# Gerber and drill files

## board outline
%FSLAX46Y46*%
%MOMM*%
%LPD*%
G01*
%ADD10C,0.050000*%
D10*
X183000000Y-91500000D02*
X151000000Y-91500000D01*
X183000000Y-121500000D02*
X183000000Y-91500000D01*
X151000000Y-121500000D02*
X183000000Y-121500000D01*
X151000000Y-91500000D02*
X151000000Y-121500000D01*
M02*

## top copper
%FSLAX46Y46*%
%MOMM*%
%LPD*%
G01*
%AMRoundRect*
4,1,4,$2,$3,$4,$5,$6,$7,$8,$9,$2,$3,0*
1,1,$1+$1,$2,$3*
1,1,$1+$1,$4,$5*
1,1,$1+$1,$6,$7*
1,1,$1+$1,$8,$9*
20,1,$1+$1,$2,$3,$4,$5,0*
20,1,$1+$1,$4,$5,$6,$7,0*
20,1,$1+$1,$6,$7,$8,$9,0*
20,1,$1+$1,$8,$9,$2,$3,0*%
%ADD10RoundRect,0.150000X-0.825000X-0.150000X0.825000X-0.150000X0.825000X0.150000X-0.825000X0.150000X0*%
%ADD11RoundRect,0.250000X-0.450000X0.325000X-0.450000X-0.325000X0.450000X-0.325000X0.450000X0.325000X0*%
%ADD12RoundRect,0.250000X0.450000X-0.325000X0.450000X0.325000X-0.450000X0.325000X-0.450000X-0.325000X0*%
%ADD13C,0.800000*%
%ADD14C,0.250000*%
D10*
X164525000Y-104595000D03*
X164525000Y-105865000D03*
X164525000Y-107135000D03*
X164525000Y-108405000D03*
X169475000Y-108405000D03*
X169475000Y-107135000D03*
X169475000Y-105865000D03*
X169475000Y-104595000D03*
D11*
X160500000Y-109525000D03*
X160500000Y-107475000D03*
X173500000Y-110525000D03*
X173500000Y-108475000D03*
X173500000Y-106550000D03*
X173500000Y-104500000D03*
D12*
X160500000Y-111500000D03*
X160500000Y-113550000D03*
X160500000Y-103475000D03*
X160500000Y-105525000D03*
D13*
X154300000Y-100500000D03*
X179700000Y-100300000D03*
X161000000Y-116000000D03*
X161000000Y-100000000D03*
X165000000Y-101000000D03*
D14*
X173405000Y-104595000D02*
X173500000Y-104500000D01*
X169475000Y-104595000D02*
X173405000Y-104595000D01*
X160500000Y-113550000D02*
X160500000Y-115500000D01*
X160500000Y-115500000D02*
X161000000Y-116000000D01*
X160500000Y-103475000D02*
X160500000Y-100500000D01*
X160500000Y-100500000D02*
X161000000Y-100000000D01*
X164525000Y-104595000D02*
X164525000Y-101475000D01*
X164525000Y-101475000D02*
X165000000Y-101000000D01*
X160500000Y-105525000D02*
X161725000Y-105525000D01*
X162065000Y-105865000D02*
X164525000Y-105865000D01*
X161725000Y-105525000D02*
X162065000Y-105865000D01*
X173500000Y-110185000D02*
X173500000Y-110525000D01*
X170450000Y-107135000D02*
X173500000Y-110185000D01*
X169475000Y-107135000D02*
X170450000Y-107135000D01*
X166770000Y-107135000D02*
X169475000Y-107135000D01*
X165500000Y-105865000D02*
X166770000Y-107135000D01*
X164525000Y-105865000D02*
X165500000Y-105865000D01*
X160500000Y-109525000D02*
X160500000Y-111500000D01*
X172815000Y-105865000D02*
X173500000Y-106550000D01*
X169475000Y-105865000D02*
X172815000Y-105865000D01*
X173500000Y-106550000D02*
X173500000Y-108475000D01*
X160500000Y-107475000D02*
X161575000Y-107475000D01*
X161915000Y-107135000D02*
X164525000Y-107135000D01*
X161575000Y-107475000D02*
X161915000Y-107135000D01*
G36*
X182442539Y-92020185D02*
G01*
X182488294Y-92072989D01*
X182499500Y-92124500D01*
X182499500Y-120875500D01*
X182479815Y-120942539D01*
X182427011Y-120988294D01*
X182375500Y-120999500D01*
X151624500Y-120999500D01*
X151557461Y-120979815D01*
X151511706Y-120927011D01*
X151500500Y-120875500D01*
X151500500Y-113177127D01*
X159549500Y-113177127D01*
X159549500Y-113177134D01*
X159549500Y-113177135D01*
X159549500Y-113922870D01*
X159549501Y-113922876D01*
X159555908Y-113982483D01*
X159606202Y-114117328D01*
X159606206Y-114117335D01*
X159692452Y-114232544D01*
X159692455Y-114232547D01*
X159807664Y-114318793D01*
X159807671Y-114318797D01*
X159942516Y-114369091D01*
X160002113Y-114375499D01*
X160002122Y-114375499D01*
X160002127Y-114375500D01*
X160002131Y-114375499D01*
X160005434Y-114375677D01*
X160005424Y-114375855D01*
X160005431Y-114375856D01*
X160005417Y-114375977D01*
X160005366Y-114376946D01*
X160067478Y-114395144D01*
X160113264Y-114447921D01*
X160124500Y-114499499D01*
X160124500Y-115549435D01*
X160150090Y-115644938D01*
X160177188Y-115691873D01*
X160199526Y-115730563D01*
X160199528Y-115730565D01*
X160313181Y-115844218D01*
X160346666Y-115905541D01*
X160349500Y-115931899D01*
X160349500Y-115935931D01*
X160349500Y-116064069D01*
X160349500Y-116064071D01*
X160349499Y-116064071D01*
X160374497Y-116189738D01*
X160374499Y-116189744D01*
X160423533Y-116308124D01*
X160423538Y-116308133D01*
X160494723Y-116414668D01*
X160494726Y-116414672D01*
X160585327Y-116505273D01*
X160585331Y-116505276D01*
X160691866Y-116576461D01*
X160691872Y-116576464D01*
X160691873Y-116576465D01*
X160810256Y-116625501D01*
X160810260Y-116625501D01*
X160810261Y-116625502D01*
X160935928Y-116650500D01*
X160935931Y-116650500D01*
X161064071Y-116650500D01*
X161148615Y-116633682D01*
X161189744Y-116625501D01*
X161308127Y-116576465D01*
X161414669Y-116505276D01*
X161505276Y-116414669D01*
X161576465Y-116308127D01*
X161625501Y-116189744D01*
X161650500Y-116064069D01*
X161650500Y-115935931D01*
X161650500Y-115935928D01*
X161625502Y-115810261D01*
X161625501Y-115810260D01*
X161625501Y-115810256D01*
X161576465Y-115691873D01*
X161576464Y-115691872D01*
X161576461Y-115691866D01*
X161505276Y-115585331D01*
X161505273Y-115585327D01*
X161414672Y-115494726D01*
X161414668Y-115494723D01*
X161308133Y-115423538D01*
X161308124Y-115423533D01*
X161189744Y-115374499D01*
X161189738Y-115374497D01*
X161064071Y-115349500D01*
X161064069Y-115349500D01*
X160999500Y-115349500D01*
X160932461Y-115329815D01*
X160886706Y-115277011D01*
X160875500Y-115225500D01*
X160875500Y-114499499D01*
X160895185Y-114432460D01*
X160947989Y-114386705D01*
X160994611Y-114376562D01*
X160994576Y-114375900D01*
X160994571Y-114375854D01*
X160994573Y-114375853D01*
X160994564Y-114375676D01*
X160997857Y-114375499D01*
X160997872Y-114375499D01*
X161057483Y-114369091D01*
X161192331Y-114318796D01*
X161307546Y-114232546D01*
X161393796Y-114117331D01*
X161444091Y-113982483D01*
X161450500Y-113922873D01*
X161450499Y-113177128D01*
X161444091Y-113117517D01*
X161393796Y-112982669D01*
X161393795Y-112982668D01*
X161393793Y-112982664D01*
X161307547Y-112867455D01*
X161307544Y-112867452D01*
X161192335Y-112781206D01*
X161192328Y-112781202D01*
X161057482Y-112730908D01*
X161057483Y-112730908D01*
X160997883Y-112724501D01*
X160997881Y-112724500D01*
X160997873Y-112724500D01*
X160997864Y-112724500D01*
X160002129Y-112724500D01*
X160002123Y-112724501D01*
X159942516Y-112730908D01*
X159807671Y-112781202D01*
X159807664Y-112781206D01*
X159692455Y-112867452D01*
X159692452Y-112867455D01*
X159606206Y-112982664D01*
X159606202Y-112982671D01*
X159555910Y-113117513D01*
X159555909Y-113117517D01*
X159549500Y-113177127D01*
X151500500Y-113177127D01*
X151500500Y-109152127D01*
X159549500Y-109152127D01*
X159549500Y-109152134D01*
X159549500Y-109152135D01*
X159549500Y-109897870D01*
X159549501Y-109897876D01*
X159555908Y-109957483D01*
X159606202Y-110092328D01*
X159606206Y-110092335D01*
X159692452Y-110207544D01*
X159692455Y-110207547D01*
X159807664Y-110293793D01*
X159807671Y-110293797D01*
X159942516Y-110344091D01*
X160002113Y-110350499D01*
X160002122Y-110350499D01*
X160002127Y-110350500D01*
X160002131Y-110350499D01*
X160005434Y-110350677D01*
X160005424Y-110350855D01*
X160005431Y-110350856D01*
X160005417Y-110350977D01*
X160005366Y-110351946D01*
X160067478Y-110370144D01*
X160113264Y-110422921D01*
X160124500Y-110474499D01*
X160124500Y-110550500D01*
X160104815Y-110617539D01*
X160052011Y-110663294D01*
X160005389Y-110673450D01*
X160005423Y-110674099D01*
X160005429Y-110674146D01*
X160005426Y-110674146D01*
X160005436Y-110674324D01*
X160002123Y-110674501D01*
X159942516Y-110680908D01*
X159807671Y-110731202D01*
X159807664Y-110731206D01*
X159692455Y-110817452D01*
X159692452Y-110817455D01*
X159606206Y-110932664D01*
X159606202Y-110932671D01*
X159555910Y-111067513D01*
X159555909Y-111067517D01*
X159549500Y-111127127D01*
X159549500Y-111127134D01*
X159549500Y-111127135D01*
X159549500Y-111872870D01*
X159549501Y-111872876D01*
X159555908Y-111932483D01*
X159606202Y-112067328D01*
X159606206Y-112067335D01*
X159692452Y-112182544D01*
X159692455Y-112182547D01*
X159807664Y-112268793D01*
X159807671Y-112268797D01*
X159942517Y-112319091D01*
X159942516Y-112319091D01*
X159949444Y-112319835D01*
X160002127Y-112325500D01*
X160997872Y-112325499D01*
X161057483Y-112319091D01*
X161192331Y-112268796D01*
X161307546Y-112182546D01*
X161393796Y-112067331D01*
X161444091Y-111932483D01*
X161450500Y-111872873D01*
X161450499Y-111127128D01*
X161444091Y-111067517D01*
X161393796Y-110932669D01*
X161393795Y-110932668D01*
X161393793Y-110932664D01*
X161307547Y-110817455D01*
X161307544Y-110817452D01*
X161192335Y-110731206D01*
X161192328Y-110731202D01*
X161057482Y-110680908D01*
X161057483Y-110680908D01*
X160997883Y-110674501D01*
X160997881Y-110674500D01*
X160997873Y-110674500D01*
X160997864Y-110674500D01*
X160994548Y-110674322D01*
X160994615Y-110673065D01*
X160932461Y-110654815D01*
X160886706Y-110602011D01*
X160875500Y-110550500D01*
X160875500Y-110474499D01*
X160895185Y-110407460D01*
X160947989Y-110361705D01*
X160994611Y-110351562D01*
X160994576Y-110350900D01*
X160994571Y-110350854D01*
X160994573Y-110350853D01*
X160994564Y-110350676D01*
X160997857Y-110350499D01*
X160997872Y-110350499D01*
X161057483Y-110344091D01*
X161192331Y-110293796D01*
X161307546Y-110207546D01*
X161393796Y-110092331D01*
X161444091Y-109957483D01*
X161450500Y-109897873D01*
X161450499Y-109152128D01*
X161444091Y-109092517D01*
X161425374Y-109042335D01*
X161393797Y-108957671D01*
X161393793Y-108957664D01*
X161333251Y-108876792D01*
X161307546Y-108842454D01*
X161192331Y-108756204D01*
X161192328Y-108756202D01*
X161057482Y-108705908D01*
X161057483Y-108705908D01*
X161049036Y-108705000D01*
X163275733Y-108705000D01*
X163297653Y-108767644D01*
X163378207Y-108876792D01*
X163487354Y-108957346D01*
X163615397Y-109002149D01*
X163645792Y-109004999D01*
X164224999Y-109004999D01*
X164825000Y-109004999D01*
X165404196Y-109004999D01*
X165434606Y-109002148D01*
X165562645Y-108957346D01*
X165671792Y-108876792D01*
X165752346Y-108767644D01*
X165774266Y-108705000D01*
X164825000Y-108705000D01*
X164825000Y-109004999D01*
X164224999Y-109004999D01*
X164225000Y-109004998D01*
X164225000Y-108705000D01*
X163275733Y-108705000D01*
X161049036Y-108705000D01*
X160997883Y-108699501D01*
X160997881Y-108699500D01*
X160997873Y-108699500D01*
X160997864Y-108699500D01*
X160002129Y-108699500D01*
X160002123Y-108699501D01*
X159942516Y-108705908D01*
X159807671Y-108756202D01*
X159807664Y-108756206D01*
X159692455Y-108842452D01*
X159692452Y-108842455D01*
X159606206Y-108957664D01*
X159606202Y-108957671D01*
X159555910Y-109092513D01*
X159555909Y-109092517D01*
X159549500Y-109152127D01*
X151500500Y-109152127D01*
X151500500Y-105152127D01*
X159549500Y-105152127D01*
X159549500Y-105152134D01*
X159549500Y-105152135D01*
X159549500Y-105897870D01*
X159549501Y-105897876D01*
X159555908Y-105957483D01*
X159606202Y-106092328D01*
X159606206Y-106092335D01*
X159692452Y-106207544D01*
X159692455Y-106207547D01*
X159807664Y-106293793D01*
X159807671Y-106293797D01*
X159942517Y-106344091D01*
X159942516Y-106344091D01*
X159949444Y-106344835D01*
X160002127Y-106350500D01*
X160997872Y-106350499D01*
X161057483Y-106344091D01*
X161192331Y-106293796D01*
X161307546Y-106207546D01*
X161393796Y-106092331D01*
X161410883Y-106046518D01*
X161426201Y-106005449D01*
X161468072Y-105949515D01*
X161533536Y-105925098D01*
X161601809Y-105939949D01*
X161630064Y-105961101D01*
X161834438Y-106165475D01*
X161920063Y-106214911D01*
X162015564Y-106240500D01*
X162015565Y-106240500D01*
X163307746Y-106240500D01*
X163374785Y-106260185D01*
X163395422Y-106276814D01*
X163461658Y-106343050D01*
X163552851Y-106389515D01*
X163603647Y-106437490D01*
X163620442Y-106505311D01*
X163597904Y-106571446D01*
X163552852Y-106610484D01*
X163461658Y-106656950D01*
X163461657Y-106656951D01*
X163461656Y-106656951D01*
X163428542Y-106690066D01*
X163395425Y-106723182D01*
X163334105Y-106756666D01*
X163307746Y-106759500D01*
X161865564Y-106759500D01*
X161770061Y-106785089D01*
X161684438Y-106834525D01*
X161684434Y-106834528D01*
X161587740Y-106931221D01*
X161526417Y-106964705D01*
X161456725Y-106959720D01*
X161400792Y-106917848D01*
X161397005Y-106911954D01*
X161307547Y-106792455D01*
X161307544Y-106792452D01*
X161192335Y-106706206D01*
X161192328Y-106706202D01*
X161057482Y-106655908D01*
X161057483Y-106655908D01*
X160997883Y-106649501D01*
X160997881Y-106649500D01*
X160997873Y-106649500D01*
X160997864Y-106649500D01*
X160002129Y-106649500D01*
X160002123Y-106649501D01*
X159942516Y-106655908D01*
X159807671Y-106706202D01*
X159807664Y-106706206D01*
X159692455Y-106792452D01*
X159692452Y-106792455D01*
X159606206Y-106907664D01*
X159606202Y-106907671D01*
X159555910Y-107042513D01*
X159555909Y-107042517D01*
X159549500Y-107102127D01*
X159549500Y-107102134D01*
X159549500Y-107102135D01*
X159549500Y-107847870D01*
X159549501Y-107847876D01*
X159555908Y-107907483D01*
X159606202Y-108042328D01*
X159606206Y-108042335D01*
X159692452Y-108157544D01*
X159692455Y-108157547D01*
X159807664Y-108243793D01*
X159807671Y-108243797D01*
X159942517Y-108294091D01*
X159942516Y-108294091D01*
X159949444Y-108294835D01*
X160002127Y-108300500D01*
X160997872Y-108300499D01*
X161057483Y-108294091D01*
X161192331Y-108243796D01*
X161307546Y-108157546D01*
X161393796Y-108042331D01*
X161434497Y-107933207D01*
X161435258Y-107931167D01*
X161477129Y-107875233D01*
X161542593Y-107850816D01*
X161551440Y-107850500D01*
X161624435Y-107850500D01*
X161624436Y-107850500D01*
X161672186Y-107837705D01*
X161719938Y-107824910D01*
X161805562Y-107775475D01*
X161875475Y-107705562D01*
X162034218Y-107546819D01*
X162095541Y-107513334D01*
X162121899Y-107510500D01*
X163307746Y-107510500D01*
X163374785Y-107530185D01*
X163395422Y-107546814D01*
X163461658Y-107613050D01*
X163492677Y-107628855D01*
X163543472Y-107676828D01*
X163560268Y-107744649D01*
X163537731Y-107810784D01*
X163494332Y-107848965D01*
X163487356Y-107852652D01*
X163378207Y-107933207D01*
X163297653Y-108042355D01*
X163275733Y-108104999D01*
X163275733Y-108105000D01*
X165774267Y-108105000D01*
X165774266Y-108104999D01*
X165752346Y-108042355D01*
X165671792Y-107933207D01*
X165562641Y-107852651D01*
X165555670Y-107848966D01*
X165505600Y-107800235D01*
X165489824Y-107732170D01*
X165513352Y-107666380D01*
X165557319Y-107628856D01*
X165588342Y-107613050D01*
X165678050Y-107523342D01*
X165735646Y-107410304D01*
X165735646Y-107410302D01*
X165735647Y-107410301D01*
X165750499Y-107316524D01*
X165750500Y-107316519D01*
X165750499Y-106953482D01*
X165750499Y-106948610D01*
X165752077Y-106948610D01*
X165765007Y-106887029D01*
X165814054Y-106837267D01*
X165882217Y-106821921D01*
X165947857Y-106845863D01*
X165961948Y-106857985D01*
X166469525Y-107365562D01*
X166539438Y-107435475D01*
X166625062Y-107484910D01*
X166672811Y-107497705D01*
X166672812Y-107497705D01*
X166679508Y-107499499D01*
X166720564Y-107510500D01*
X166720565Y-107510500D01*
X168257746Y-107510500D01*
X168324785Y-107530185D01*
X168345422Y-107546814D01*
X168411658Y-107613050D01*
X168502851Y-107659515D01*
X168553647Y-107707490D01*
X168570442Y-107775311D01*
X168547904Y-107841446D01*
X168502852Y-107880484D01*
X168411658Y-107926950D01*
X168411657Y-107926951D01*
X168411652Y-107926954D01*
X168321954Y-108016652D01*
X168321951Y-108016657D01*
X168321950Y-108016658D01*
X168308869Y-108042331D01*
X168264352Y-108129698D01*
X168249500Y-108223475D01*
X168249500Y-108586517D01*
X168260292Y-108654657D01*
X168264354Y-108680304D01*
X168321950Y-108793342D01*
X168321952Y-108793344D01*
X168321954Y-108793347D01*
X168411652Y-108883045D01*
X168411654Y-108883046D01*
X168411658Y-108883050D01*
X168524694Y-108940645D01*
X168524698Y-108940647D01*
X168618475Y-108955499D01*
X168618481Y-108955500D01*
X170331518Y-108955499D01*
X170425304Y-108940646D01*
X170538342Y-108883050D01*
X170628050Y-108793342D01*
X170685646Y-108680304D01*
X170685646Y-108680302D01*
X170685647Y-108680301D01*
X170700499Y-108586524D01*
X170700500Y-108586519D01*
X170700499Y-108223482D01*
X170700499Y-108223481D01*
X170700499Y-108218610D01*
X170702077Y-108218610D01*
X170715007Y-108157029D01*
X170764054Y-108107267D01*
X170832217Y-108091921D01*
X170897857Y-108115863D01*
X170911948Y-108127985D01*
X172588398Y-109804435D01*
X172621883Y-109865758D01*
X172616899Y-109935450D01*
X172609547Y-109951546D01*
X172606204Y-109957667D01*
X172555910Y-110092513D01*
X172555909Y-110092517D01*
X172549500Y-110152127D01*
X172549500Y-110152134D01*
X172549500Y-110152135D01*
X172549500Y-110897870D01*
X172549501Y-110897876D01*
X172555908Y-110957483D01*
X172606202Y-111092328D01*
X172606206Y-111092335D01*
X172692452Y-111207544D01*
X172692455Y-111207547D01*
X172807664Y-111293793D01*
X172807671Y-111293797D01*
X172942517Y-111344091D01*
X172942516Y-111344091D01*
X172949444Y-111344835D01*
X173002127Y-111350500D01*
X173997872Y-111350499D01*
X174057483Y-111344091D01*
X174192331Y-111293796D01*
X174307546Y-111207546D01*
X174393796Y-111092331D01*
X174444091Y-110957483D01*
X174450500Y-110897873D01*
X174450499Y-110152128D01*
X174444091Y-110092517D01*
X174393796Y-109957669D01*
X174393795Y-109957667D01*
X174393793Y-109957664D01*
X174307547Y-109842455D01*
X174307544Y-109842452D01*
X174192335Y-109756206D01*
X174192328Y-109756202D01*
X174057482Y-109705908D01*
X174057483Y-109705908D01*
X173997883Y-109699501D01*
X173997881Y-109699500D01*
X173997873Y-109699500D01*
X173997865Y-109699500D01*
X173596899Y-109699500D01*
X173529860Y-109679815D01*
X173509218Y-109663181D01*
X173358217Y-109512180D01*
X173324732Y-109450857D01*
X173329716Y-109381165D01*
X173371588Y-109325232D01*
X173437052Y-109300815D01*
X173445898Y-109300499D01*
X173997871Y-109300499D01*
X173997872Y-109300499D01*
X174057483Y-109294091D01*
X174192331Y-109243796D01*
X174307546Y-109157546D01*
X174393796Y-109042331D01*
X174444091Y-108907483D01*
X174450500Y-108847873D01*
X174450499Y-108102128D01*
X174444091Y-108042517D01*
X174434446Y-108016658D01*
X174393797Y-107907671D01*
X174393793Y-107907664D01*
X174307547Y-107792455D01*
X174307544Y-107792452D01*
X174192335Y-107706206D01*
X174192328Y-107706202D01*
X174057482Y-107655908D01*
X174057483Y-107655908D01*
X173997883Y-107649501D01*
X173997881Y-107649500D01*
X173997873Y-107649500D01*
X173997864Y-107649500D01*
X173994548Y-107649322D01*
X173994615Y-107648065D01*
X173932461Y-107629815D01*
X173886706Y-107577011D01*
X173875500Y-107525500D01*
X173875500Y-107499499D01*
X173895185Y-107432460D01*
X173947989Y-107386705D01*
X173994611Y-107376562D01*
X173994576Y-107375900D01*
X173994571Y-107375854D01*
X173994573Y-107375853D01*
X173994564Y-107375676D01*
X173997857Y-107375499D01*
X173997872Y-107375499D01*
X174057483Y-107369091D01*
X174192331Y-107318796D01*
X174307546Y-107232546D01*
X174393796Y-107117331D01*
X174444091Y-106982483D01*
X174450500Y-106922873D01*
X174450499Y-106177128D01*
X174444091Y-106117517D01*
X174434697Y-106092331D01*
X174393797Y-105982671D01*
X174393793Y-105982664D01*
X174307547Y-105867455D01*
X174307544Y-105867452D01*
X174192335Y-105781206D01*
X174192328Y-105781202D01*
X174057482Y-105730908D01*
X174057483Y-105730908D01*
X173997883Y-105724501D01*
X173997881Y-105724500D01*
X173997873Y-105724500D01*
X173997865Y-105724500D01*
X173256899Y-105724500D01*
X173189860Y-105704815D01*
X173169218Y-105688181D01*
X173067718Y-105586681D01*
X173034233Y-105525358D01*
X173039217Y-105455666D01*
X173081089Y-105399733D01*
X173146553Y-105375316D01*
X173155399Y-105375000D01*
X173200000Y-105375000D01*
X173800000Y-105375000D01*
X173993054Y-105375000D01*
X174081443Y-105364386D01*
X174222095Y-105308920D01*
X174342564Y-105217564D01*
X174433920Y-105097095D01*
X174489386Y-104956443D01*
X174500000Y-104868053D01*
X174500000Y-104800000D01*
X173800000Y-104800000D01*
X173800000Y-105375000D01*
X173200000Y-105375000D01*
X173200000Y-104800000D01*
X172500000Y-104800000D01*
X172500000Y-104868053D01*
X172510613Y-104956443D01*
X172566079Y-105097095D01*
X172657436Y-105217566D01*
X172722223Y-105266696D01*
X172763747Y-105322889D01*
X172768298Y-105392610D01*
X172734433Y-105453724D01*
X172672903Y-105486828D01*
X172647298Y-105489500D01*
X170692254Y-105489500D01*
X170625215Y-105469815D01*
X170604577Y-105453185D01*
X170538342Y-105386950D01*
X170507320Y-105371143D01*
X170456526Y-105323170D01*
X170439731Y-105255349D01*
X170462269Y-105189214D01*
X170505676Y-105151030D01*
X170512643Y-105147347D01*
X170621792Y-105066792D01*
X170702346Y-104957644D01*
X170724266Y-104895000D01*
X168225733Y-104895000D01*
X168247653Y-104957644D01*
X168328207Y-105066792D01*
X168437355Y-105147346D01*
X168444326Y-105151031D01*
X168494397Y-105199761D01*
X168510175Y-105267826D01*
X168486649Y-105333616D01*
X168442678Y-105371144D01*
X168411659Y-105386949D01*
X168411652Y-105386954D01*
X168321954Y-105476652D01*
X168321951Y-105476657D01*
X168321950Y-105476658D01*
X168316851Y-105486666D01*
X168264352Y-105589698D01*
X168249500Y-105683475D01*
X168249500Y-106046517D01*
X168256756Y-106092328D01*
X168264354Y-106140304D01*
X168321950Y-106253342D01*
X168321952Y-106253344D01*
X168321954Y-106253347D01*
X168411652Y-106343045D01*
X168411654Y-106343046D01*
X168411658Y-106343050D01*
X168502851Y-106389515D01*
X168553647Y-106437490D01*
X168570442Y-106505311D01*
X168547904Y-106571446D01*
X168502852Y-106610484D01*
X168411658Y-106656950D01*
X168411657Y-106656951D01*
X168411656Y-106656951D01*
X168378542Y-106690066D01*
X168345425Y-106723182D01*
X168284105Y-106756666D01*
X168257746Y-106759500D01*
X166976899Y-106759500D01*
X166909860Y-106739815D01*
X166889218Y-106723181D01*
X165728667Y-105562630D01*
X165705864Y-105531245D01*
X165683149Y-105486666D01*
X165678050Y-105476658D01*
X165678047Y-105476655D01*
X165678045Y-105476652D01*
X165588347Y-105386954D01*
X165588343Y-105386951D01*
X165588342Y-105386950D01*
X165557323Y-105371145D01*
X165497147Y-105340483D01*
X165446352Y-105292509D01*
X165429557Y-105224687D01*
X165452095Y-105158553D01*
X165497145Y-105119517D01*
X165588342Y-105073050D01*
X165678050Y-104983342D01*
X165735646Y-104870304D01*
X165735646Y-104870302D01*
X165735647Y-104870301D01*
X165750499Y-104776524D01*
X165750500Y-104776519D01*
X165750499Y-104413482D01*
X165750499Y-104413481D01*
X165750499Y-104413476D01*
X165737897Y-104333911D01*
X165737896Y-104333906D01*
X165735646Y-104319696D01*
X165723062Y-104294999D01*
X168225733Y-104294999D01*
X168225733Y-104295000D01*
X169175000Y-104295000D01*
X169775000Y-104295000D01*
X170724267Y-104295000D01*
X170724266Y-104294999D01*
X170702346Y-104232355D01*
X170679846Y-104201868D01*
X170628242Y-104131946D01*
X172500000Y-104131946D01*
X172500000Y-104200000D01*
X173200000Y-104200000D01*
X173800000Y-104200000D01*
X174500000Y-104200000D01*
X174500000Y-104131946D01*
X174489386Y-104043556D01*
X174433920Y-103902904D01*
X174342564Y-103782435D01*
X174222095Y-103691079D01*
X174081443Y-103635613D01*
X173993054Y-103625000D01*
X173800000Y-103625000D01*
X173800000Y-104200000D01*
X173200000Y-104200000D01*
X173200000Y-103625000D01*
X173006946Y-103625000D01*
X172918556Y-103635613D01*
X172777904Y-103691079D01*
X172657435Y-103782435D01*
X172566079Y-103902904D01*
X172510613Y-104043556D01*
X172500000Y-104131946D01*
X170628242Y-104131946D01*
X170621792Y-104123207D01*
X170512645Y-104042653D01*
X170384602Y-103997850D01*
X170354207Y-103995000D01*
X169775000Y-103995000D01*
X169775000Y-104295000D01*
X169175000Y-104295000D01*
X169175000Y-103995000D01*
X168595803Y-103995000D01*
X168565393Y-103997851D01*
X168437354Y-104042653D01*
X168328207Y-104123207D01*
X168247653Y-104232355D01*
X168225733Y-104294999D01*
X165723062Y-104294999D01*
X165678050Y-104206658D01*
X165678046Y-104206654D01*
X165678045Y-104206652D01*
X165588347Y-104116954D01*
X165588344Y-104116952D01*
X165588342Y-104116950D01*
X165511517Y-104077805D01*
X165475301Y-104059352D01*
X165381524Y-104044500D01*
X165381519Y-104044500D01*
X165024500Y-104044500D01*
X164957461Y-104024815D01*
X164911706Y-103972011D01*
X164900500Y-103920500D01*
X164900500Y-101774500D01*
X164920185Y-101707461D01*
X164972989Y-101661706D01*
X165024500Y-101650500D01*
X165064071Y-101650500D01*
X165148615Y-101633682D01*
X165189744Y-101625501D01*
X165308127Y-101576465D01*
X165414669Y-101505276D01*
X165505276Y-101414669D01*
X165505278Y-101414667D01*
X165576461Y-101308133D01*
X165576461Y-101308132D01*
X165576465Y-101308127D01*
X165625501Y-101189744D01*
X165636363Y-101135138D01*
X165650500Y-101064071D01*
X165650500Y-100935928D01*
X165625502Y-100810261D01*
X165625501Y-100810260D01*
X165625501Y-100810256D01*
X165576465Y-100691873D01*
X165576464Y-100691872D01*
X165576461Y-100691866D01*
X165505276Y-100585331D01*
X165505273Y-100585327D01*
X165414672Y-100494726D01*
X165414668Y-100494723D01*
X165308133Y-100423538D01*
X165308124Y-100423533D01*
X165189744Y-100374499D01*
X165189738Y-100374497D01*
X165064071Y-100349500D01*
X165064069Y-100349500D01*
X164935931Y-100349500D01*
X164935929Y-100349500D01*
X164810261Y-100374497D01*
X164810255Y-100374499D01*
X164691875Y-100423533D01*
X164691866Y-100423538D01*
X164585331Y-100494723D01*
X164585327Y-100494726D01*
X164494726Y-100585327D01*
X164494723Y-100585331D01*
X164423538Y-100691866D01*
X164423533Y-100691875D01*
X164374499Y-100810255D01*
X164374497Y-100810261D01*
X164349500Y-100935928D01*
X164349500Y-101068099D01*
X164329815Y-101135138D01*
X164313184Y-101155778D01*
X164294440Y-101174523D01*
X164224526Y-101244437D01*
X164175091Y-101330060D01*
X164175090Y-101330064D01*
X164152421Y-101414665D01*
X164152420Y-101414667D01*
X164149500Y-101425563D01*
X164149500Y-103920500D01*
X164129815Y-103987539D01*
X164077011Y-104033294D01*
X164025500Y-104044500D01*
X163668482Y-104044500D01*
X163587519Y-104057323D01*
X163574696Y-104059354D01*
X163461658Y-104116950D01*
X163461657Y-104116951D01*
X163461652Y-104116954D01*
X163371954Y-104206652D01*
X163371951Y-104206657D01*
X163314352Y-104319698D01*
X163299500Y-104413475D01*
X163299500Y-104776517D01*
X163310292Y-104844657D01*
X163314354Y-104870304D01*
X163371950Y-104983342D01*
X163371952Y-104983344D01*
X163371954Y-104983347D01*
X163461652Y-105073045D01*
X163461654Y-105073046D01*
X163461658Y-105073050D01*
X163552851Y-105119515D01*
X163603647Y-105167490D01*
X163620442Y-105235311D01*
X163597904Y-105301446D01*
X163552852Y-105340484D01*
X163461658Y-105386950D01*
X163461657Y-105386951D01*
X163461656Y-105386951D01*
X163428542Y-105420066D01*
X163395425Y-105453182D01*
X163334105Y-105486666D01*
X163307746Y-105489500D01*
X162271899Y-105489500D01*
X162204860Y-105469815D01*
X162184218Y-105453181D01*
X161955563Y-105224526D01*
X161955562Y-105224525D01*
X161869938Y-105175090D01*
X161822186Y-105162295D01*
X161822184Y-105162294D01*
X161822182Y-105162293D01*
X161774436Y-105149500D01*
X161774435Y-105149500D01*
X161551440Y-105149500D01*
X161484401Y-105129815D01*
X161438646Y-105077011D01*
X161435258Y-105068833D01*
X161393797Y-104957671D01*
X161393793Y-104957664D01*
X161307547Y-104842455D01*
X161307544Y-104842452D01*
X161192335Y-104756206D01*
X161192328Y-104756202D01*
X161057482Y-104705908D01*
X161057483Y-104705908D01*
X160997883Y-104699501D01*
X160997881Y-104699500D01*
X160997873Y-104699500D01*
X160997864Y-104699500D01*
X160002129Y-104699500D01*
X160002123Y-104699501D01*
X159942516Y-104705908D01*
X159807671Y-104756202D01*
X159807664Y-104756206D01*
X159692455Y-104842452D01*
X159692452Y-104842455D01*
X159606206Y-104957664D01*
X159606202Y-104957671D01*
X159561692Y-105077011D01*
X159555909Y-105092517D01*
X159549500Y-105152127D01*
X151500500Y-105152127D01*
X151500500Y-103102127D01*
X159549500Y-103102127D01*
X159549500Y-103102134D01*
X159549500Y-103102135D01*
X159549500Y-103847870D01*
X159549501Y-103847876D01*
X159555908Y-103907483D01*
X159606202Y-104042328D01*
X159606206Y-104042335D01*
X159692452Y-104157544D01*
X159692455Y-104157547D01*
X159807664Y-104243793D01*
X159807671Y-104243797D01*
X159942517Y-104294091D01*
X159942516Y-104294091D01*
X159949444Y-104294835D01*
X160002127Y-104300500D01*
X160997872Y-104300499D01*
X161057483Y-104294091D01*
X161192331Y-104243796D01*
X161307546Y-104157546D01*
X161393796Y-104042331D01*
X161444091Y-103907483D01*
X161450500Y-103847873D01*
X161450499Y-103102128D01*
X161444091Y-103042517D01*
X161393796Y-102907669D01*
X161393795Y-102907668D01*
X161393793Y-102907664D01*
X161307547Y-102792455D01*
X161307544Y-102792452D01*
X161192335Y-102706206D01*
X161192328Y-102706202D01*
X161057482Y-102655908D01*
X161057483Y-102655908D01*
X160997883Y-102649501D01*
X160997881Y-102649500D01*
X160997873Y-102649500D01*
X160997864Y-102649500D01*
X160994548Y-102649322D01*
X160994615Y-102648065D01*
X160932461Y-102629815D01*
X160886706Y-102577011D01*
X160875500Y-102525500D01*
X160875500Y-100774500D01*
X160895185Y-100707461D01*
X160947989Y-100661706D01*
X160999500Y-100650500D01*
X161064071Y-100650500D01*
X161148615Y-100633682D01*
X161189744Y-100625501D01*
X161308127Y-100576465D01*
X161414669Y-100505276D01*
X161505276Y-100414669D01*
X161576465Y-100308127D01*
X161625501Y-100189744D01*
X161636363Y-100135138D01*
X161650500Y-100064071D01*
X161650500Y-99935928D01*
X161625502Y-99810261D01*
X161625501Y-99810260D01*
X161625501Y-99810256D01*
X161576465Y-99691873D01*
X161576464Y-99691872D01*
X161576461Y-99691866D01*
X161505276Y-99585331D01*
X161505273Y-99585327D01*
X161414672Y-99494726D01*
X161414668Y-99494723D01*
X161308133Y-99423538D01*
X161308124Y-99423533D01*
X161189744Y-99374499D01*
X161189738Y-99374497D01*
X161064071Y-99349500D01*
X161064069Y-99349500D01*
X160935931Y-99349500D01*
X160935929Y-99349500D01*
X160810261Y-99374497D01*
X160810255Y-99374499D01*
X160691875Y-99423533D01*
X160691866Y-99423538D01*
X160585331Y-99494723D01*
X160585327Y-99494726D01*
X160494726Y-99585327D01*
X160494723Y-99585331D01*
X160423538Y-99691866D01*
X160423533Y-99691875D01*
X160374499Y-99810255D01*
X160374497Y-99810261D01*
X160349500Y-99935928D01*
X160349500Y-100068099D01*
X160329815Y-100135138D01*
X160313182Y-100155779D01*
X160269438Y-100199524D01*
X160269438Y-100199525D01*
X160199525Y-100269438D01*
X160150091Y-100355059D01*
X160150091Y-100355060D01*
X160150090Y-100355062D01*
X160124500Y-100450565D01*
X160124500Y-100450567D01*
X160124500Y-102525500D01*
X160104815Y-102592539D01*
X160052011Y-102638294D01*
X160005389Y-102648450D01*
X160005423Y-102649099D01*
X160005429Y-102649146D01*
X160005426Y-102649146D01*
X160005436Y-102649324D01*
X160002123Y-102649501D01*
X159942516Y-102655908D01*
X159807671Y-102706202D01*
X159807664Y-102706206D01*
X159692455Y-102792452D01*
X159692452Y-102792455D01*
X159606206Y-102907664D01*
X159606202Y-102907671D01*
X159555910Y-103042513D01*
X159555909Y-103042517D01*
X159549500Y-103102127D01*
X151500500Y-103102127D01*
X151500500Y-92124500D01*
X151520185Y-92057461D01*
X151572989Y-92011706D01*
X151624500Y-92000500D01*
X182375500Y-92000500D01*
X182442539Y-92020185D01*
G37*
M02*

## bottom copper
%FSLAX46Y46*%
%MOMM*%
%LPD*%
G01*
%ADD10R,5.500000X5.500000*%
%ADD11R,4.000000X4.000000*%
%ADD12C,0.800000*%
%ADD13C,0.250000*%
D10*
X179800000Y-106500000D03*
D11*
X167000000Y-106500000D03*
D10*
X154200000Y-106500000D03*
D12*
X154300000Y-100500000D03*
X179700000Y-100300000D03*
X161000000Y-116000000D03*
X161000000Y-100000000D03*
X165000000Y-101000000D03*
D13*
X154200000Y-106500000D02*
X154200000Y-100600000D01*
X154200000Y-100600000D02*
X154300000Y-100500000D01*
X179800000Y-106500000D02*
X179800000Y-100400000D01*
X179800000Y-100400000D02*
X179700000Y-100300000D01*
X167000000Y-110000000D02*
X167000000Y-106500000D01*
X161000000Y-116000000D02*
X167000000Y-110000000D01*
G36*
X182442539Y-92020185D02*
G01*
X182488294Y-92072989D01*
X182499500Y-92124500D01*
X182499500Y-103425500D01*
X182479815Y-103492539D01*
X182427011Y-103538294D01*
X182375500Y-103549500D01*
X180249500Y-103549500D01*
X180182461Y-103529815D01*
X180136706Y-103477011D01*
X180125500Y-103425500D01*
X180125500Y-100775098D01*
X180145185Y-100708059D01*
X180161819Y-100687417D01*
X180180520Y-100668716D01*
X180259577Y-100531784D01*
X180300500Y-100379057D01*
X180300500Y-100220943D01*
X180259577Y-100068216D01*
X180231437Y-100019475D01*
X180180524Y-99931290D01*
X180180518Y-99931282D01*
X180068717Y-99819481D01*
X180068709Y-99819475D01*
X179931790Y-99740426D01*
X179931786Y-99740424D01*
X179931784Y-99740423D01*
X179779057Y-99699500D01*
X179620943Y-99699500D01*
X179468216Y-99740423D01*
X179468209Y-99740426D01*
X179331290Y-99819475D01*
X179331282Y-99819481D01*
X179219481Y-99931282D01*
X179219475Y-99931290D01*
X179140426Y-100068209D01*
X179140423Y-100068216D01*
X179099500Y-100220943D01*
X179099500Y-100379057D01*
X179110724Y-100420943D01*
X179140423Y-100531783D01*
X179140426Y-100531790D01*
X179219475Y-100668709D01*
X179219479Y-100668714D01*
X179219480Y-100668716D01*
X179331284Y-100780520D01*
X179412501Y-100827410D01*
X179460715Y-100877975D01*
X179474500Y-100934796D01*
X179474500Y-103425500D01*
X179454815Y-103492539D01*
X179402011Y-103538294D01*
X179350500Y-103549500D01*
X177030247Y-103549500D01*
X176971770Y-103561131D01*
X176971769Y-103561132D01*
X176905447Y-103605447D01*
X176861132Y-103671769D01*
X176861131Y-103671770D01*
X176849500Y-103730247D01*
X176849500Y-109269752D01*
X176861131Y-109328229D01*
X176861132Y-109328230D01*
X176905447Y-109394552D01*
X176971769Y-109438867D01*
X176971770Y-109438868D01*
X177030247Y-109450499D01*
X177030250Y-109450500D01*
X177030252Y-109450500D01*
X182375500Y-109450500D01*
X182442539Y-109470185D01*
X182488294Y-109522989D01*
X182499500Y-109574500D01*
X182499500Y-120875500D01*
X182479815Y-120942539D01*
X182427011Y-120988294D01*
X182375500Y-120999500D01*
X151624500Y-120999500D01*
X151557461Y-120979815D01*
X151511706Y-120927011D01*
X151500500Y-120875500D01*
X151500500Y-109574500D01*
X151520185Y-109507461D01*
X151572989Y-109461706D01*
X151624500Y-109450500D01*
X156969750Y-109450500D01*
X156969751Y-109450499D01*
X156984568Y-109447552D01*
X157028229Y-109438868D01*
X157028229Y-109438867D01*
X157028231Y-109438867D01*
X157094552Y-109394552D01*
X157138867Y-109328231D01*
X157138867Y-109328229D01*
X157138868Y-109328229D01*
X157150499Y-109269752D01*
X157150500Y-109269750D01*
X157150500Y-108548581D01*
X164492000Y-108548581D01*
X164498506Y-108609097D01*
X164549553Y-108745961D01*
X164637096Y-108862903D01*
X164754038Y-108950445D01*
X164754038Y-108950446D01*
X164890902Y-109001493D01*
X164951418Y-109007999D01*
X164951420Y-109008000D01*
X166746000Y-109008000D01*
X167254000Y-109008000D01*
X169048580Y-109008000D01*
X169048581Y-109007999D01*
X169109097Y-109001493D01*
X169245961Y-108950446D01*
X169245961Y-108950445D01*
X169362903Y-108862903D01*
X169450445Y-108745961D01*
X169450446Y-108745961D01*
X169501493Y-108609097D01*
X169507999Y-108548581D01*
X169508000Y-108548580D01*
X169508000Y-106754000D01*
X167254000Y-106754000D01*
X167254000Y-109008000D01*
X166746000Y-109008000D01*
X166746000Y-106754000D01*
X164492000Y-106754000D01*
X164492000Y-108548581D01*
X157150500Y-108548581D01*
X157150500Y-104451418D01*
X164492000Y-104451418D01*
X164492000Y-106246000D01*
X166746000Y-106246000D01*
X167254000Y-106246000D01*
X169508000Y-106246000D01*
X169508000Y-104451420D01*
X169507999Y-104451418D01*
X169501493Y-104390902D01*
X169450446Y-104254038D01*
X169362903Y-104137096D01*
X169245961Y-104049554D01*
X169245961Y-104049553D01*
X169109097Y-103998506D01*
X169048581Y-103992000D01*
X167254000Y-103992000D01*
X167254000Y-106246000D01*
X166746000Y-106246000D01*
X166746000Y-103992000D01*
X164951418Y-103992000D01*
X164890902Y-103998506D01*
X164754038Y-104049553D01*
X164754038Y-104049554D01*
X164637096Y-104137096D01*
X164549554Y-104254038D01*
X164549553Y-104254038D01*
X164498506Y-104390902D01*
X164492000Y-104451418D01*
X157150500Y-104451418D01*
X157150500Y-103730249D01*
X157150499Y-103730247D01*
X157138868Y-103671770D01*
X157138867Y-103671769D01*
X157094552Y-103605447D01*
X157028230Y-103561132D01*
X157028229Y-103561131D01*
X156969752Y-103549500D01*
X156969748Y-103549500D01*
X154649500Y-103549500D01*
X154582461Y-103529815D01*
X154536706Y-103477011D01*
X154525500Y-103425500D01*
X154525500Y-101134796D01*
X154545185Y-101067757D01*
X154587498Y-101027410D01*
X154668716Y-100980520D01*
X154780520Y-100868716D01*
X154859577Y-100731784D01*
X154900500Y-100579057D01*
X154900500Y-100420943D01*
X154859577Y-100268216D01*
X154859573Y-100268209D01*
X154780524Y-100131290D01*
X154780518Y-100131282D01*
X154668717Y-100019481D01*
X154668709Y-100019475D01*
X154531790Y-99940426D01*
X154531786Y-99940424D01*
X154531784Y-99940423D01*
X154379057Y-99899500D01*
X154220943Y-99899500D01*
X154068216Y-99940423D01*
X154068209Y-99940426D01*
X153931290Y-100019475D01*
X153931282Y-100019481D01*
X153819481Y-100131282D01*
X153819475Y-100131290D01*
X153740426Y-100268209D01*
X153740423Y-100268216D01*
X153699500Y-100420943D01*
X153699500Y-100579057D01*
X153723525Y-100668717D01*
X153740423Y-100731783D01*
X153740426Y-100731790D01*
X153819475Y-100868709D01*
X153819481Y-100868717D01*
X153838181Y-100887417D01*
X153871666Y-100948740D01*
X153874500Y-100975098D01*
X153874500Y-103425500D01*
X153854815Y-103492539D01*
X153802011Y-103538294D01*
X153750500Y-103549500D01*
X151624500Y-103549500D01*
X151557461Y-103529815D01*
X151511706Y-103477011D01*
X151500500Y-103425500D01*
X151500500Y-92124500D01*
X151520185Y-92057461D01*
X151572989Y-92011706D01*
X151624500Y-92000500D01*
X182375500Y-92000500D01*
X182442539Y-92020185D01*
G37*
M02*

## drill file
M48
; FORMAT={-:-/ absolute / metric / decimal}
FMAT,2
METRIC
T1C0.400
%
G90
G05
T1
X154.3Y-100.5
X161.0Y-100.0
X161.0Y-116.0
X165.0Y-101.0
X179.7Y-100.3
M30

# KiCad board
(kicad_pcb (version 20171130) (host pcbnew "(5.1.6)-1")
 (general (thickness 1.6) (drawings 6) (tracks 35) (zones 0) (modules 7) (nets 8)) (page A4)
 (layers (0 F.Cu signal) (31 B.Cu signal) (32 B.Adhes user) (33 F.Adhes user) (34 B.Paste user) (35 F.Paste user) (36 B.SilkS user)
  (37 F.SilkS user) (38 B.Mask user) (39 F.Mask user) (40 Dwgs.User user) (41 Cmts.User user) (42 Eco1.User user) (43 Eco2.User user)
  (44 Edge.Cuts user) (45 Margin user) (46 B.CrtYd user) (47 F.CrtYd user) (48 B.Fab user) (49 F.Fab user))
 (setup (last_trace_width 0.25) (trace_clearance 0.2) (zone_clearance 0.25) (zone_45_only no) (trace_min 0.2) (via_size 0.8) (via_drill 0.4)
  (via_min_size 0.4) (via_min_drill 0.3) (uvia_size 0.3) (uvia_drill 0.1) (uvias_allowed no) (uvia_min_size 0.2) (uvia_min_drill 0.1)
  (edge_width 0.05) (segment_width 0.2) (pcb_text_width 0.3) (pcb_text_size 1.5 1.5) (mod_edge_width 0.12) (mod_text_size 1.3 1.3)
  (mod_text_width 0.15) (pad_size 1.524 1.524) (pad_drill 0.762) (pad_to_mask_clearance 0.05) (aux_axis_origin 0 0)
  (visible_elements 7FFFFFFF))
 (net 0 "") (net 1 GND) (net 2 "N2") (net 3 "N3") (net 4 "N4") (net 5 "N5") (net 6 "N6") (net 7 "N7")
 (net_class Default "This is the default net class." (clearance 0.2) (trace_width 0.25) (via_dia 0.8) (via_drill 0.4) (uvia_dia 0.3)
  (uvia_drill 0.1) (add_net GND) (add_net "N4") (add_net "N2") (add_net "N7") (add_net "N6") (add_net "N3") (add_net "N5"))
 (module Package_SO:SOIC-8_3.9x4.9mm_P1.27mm (layer F.Cu) (at 167 106.5)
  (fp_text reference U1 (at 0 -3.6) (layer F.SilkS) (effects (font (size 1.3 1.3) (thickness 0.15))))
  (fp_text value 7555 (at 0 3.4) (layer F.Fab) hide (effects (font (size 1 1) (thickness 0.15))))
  (pad 1 smd roundrect (at -2.475 -1.905) (size 1.95 0.6) (layers F.Cu F.Paste F.Mask) (roundrect_rratio 0.25) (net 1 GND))
  (pad 2 smd roundrect (at -2.475 -0.635) (size 1.95 0.6) (layers F.Cu F.Paste F.Mask) (roundrect_rratio 0.25) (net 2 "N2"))
  (pad 3 smd roundrect (at -2.475 0.635) (size 1.95 0.6) (layers F.Cu F.Paste F.Mask) (roundrect_rratio 0.25) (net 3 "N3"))
  (pad 4 smd roundrect (at -2.475 1.905) (size 1.95 0.6) (layers F.Cu F.Paste F.Mask) (roundrect_rratio 0.25) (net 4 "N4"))
  (pad 5 smd roundrect (at 2.475 1.905) (size 1.95 0.6) (layers F.Cu F.Paste F.Mask) (roundrect_rratio 0.25) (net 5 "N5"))
  (pad 6 smd roundrect (at 2.475 0.635) (size 1.95 0.6) (layers F.Cu F.Paste F.Mask) (roundrect_rratio 0.25) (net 2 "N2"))
  (pad 7 smd roundrect (at 2.475 -0.635) (size 1.95 0.6) (layers F.Cu F.Paste F.Mask) (roundrect_rratio 0.25) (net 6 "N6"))
  (pad 8 smd roundrect (at 2.475 -1.905) (size 1.95 0.6) (layers F.Cu F.Paste F.Mask) (roundrect_rratio 0.25) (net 4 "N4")))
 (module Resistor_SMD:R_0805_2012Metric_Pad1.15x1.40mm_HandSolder (layer F.Cu) (at 160.5 108.5 270)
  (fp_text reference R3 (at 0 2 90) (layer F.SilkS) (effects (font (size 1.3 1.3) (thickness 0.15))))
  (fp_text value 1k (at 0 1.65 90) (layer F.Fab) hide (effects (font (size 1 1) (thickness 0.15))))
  (pad 2 smd roundrect (at 1.025 0 270) (size 1.15 1.4) (layers F.Cu F.Paste F.Mask) (roundrect_rratio 0.217391) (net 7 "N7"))
  (pad 1 smd roundrect (at -1.025 0 270) (size 1.15 1.4) (layers F.Cu F.Paste F.Mask) (roundrect_rratio 0.217391) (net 3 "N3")))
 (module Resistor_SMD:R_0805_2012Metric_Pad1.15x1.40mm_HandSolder (layer F.Cu) (at 173.5 109.5 270)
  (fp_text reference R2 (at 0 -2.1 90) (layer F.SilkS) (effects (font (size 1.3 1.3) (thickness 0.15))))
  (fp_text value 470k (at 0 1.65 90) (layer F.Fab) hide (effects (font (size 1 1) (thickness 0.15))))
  (pad 2 smd roundrect (at 1.025 0 270) (size 1.15 1.4) (layers F.Cu F.Paste F.Mask) (roundrect_rratio 0.217391) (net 2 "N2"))
  (pad 1 smd roundrect (at -1.025 0 270) (size 1.15 1.4) (layers F.Cu F.Paste F.Mask) (roundrect_rratio 0.217391) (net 6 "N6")))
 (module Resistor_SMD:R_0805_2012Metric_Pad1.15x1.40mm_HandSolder (layer F.Cu) (at 173.5 105.525 270)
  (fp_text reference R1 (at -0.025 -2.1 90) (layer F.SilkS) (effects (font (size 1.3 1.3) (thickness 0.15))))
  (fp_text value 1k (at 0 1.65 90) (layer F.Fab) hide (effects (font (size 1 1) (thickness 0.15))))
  (pad 2 smd roundrect (at 1.025 0 270) (size 1.15 1.4) (layers F.Cu F.Paste F.Mask) (roundrect_rratio 0.217391) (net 6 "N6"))
  (pad 1 smd roundrect (at -1.025 0 270) (size 1.15 1.4) (layers F.Cu F.Paste F.Mask) (roundrect_rratio 0.217391) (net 4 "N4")))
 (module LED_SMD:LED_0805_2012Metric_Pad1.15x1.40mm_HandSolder (layer F.Cu) (at 160.5 112.525 90)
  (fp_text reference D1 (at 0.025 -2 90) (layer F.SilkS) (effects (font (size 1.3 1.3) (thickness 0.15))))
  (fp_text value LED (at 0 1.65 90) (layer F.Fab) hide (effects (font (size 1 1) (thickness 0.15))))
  (pad 2 smd roundrect (at 1.025 0 90) (size 1.15 1.4) (layers F.Cu F.Paste F.Mask) (roundrect_rratio 0.217391) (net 7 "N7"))
  (pad 1 smd roundrect (at -1.025 0 90) (size 1.15 1.4) (layers F.Cu F.Paste F.Mask) (roundrect_rratio 0.217391) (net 1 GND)))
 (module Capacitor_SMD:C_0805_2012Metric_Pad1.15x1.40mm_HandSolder (layer F.Cu) (at 160.5 104.5 90)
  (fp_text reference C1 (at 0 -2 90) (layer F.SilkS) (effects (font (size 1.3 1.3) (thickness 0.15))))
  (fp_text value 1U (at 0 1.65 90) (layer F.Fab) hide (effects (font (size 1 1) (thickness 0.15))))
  (pad 2 smd roundrect (at 1.025 0 90) (size 1.15 1.4) (layers F.Cu F.Paste F.Mask) (roundrect_rratio 0.217391) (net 1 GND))
  (pad 1 smd roundrect (at -1.025 0 90) (size 1.15 1.4) (layers F.Cu F.Paste F.Mask) (roundrect_rratio 0.217391) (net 2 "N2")))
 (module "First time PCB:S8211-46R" (layer B.Cu) (at 167 106.5)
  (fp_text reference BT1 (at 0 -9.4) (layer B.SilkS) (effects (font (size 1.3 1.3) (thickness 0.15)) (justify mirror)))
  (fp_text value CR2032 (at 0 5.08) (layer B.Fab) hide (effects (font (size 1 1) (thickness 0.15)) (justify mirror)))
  (pad 1 smd rect (at 12.8 0) (size 5.5 5.5) (layers B.Cu B.Paste B.Mask) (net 4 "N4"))
  (pad 2 smd rect (at 0 0) (size 4 4) (layers B.Cu B.Paste B.Mask) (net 1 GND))
  (pad 1 smd rect (at -12.8 0) (size 5.5 5.5) (layers B.Cu B.Paste B.Mask) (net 4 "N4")))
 (gr_line (start 183 91.5) (end 151 91.5) (layer Edge.Cuts) (width 0.05))
 (gr_line (start 183 121.5) (end 183 91.5) (layer Edge.Cuts) (width 0.05))
 (gr_line (start 151 121.5) (end 183 121.5) (layer Edge.Cuts) (width 0.05))
 (gr_line (start 151 91.5) (end 151 121.5) (layer Edge.Cuts) (width 0.05))
 (segment (start 173.405 104.595) (end 173.5 104.5) (width 0.25) (layer F.Cu) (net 4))
 (segment (start 169.475 104.595) (end 173.405 104.595) (width 0.25) (layer F.Cu) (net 4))
 (segment (start 154.2 106.5) (end 154.2 100.6) (width 0.25) (layer B.Cu) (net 4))
 (via (at 154.3 100.5) (size 0.8) (drill 0.4) (layers F.Cu B.Cu) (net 4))
 (segment (start 154.2 100.6) (end 154.3 100.5) (width 0.25) (layer B.Cu) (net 4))
 (via (at 179.7 100.3) (size 0.8) (drill 0.4) (layers F.Cu B.Cu) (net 4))
 (segment (start 179.8 106.5) (end 179.8 100.4) (width 0.25) (layer B.Cu) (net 4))
 (segment (start 179.8 100.4) (end 179.7 100.3) (width 0.25) (layer B.Cu) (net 4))
 (via (at 161 116) (size 0.8) (drill 0.4) (layers F.Cu B.Cu) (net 1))
 (segment (start 160.5 113.55) (end 160.5 115.5) (width 0.25) (layer F.Cu) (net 1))
 (segment (start 160.5 115.5) (end 161 116) (width 0.25) (layer F.Cu) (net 1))
 (segment (start 167 110) (end 167 106.5) (width 0.25) (layer B.Cu) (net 1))
 (segment (start 161 116) (end 167 110) (width 0.25) (layer B.Cu) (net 1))
 (segment (start 160.5 103.475) (end 160.5 100.5) (width 0.25) (layer F.Cu) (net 1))
 (via (at 161 100) (size 0.8) (drill 0.4) (layers F.Cu B.Cu) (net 1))
 (segment (start 160.5 100.5) (end 161 100) (width 0.25) (layer F.Cu) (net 1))
 (via (at 165 101) (size 0.8) (drill 0.4) (layers F.Cu B.Cu) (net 1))
 (segment (start 164.525 104.595) (end 164.525 101.475) (width 0.25) (layer F.Cu) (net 1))
 (segment (start 164.525 101.475) (end 165 101) (width 0.25) (layer F.Cu) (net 1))
 (segment (start 160.5 105.525) (end 161.725 105.525) (width 0.25) (layer F.Cu) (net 2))
 (segment (start 162.065 105.865) (end 164.525 105.865) (width 0.25) (layer F.Cu) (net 2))
 (segment (start 161.725 105.525) (end 162.065 105.865) (width 0.25) (layer F.Cu) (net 2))
 (segment (start 173.5 110.185) (end 173.5 110.525) (width 0.25) (layer F.Cu) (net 2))
 (segment (start 170.45 107.135) (end 173.5 110.185) (width 0.25) (layer F.Cu) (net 2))
 (segment (start 169.475 107.135) (end 170.45 107.135) (width 0.25) (layer F.Cu) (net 2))
 (segment (start 166.77 107.135) (end 169.475 107.135) (width 0.25) (layer F.Cu) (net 2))
 (segment (start 165.5 105.865) (end 166.77 107.135) (width 0.25) (layer F.Cu) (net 2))
 (segment (start 164.525 105.865) (end 165.5 105.865) (width 0.25) (layer F.Cu) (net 2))
 (segment (start 160.5 109.525) (end 160.5 111.5) (width 0.25) (layer F.Cu) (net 7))
 (segment (start 172.815 105.865) (end 173.5 106.55) (width 0.25) (layer F.Cu) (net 6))
 (segment (start 169.475 105.865) (end 172.815 105.865) (width 0.25) (layer F.Cu) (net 6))
 (segment (start 173.5 106.55) (end 173.5 108.475) (width 0.25) (layer F.Cu) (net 6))
 (segment (start 160.5 107.475) (end 161.575 107.475) (width 0.25) (layer F.Cu) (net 3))
 (segment (start 161.915 107.135) (end 164.525 107.135) (width 0.25) (layer F.Cu) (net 3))
 (segment (start 161.575 107.475) (end 161.915 107.135) (width 0.25) (layer F.Cu) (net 3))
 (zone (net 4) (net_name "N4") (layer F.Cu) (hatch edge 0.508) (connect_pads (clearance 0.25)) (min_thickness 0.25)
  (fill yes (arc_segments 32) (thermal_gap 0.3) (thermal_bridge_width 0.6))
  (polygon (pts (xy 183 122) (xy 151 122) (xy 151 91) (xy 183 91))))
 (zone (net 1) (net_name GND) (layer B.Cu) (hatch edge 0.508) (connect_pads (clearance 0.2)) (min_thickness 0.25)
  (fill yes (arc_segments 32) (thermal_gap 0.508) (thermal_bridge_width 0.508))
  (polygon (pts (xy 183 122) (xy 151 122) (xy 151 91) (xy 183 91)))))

